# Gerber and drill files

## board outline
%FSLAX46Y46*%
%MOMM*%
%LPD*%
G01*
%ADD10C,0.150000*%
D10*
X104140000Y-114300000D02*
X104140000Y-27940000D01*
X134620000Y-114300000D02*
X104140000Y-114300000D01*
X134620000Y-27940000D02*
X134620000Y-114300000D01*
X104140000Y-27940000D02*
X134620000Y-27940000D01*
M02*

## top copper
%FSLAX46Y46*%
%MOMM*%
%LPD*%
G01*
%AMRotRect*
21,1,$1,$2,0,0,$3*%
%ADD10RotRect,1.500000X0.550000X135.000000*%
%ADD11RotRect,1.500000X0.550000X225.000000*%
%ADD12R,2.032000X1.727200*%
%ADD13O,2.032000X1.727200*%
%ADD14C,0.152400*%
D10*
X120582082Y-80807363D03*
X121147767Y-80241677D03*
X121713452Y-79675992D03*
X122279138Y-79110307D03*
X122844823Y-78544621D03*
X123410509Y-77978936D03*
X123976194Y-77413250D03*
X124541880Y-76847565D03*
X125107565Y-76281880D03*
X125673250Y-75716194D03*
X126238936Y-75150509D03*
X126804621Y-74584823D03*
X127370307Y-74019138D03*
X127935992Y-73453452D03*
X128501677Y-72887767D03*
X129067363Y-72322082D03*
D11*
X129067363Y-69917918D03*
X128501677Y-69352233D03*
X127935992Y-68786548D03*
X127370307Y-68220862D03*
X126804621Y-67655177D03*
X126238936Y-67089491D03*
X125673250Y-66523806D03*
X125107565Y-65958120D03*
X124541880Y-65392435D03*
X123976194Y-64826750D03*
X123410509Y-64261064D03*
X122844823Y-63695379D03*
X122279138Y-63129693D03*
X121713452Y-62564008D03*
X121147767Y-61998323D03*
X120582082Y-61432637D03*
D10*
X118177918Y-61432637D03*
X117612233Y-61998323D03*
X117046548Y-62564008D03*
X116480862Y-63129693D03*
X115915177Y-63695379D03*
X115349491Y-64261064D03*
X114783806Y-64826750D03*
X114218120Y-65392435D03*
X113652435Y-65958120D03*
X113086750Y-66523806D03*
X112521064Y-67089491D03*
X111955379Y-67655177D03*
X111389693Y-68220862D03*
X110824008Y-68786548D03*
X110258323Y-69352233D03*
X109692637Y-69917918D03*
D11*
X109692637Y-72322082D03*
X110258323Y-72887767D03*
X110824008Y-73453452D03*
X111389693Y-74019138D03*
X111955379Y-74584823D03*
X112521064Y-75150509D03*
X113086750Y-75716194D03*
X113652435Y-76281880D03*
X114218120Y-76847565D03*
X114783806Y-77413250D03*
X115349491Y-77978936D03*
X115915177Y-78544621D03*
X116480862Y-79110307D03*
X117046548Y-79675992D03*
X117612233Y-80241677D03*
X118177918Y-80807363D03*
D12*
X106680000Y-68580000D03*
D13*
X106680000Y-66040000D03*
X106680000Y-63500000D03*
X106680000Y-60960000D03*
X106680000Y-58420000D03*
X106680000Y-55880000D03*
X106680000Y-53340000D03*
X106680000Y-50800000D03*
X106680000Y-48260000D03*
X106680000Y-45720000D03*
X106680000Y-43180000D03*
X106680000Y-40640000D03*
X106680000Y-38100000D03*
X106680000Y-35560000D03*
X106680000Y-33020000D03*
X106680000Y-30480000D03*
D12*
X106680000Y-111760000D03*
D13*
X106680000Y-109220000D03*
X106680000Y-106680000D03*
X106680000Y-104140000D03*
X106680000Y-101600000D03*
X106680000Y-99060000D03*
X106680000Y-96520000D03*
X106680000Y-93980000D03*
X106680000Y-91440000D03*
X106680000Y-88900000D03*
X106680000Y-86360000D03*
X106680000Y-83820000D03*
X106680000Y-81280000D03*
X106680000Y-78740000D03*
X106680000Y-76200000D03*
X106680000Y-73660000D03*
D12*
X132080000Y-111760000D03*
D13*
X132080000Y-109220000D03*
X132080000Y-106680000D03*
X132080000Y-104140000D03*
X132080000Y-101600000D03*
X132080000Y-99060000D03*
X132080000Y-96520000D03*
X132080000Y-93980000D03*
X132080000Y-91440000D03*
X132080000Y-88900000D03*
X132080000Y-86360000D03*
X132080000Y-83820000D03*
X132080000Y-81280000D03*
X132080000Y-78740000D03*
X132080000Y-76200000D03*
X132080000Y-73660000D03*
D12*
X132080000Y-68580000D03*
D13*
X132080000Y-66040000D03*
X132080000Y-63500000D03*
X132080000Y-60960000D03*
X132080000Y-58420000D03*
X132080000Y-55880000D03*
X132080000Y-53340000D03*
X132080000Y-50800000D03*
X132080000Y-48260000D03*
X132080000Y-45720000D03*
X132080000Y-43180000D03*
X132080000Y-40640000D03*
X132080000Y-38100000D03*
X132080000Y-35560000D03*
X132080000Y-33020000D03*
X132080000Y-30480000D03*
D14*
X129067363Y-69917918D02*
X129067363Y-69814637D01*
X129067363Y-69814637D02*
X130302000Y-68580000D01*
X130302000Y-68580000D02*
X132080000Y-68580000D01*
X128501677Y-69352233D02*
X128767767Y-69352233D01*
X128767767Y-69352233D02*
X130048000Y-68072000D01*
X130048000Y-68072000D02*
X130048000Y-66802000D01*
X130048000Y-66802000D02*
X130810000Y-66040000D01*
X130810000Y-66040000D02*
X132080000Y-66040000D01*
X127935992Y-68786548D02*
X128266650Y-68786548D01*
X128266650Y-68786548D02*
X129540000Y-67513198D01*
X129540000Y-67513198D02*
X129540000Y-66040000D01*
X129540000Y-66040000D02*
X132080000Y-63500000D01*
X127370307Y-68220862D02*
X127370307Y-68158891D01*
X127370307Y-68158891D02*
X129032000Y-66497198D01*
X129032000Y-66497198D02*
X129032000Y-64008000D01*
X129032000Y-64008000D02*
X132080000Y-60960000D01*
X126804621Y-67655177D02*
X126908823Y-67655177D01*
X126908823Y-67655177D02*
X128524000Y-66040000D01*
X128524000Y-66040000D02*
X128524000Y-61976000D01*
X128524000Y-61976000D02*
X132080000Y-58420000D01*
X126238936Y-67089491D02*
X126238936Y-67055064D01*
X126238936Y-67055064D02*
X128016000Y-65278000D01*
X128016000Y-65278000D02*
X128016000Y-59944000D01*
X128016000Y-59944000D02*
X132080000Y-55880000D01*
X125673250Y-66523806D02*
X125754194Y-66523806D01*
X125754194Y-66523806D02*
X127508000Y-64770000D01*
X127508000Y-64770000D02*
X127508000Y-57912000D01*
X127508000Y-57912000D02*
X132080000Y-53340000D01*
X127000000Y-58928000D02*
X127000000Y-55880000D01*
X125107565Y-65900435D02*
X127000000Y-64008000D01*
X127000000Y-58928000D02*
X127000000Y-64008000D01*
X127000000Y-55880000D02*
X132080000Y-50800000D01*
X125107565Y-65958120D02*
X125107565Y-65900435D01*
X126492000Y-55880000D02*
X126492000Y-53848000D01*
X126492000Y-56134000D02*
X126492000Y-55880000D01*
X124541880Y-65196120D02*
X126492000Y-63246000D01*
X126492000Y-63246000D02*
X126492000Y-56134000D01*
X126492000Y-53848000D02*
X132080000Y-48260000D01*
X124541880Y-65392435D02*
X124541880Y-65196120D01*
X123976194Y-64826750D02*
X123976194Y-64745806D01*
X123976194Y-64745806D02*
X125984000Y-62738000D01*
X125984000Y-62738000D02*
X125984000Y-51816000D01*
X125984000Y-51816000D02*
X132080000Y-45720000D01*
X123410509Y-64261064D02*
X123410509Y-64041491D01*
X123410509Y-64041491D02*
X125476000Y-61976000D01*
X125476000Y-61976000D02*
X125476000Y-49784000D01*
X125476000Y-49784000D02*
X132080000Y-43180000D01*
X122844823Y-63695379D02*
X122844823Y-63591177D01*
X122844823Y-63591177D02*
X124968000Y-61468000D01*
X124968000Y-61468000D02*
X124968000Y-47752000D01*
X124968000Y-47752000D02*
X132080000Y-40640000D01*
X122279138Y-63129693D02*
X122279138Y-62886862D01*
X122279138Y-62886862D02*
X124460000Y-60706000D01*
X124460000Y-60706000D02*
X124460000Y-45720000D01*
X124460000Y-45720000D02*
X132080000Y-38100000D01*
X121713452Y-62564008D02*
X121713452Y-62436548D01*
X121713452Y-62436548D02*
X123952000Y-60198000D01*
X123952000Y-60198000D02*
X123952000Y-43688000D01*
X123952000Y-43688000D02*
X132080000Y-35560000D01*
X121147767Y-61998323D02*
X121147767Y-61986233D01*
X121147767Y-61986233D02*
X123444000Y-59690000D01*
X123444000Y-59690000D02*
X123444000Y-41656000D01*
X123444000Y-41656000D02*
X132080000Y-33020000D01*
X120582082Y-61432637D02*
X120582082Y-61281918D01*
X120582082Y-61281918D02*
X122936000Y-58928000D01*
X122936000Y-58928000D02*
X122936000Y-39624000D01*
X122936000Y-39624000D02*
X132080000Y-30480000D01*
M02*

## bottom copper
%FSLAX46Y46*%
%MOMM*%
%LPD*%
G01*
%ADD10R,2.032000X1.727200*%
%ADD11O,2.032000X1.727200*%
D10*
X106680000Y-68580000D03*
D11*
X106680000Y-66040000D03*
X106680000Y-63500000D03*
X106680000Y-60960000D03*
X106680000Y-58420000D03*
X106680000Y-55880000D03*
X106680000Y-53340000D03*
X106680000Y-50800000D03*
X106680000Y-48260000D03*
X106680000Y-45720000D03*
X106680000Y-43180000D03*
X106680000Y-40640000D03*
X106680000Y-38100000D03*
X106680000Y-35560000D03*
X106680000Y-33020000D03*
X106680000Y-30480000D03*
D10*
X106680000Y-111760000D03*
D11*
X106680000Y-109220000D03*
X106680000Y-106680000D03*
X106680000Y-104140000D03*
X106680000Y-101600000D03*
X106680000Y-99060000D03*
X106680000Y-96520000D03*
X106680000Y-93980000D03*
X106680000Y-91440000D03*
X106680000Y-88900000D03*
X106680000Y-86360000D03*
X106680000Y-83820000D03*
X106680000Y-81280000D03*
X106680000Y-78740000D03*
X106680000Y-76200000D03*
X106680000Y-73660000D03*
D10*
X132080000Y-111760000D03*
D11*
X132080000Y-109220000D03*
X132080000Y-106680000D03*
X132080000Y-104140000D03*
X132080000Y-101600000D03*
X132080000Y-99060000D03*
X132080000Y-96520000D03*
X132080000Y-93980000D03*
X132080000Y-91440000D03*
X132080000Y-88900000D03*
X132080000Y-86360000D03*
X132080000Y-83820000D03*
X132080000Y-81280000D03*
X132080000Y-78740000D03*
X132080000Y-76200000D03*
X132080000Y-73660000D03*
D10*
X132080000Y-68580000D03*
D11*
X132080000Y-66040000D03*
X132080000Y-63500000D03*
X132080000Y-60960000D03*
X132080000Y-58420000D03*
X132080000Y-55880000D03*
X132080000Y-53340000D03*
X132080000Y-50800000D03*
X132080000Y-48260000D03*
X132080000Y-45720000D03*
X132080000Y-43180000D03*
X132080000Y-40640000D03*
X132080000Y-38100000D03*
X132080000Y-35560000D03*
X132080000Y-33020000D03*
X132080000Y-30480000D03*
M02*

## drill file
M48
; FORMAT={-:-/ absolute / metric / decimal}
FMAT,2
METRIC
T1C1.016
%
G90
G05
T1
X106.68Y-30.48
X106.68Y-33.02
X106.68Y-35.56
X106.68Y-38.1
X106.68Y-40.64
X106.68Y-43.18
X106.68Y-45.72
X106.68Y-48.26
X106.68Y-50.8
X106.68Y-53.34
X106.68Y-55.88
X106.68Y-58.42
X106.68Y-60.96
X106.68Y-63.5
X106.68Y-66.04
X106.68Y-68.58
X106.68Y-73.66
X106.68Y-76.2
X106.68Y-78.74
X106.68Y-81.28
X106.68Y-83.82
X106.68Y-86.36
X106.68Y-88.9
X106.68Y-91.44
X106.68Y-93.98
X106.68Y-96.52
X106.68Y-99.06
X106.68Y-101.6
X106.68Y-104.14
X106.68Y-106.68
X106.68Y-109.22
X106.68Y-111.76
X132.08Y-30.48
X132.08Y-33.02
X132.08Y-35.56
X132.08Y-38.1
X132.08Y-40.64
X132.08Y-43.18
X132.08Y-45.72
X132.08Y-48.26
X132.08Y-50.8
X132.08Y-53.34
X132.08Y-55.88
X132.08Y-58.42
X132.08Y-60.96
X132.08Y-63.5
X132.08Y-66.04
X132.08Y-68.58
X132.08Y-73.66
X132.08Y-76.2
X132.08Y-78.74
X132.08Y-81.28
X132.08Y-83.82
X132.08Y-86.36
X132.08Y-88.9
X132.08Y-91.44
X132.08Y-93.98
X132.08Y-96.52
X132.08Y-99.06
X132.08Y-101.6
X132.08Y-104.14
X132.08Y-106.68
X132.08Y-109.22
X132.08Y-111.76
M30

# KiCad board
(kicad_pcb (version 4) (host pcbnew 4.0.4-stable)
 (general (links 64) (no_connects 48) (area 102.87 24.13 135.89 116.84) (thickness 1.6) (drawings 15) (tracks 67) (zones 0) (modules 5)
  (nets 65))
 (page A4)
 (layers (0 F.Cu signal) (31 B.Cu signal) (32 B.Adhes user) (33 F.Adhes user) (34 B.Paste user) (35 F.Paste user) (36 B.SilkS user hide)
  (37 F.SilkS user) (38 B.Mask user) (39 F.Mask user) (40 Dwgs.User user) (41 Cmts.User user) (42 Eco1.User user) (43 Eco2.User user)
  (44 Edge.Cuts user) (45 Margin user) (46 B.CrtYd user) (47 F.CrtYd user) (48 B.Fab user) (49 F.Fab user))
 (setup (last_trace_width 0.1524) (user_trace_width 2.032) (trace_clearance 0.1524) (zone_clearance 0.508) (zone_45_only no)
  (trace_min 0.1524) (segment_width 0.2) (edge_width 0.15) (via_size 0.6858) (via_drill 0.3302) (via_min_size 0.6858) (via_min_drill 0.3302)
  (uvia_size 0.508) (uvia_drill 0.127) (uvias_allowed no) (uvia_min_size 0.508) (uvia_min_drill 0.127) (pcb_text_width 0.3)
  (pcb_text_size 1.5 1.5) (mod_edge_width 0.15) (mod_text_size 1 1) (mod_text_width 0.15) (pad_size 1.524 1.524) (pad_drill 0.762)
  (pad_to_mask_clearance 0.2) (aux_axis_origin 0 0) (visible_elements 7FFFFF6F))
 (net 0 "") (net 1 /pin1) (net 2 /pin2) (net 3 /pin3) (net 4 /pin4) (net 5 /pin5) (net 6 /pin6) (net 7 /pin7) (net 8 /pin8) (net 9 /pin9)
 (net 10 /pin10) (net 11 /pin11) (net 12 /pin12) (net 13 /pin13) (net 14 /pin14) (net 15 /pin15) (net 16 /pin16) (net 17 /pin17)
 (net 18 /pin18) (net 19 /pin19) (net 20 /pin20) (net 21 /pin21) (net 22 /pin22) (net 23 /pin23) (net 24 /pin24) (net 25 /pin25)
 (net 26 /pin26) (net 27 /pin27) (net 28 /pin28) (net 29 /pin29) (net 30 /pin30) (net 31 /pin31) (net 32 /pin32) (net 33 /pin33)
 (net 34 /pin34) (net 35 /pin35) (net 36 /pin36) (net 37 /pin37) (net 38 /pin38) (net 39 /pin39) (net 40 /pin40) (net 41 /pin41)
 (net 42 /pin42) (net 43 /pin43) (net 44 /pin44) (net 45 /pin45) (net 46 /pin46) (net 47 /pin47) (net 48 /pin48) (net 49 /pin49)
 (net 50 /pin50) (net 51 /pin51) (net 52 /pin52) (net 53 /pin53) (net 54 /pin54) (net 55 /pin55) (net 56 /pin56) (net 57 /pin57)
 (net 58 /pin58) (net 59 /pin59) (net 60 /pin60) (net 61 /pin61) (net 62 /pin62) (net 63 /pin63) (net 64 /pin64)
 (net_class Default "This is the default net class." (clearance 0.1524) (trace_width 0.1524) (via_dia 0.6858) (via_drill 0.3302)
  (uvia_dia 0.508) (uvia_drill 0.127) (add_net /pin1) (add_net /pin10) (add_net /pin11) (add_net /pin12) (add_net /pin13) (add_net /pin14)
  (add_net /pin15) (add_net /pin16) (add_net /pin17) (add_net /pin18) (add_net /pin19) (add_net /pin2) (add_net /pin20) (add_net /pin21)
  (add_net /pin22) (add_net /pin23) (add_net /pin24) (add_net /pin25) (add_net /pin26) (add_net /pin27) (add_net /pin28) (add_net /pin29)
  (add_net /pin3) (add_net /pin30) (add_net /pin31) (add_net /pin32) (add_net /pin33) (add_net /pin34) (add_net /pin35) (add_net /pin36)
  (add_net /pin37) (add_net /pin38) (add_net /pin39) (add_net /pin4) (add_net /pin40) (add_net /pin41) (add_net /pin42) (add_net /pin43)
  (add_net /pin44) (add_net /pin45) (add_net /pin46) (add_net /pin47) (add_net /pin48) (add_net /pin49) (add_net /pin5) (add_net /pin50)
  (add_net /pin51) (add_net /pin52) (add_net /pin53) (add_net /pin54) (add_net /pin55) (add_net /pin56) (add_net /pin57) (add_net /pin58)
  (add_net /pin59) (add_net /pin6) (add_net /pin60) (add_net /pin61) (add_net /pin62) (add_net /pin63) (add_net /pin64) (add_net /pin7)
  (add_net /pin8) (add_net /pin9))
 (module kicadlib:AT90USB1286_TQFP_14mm (layer F.Cu) (at 119.38 71.12 135)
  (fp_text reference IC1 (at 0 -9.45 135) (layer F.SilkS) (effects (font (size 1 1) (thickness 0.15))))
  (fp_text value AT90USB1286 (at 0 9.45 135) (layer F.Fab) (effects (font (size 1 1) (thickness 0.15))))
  (pad 1 smd rect (at -7.7 -6 135) (size 1.5 0.55) (layers F.Cu F.Paste F.Mask) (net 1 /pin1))
  (pad 2 smd rect (at -7.7 -5.2 135) (size 1.5 0.55) (layers F.Cu F.Paste F.Mask) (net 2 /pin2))
  (pad 3 smd rect (at -7.7 -4.4 135) (size 1.5 0.55) (layers F.Cu F.Paste F.Mask) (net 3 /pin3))
  (pad 4 smd rect (at -7.7 -3.6 135) (size 1.5 0.55) (layers F.Cu F.Paste F.Mask) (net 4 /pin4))
  (pad 5 smd rect (at -7.7 -2.8 135) (size 1.5 0.55) (layers F.Cu F.Paste F.Mask) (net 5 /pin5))
  (pad 6 smd rect (at -7.7 -2 135) (size 1.5 0.55) (layers F.Cu F.Paste F.Mask) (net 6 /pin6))
  (pad 7 smd rect (at -7.7 -1.2 135) (size 1.5 0.55) (layers F.Cu F.Paste F.Mask) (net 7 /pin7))
  (pad 8 smd rect (at -7.7 -0.4 135) (size 1.5 0.55) (layers F.Cu F.Paste F.Mask) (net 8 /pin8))
  (pad 9 smd rect (at -7.7 0.4 135) (size 1.5 0.55) (layers F.Cu F.Paste F.Mask) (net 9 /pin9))
  (pad 10 smd rect (at -7.7 1.2 135) (size 1.5 0.55) (layers F.Cu F.Paste F.Mask) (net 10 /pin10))
  (pad 11 smd rect (at -7.7 2 135) (size 1.5 0.55) (layers F.Cu F.Paste F.Mask) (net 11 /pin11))
  (pad 12 smd rect (at -7.7 2.8 135) (size 1.5 0.55) (layers F.Cu F.Paste F.Mask) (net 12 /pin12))
  (pad 13 smd rect (at -7.7 3.6 135) (size 1.5 0.55) (layers F.Cu F.Paste F.Mask) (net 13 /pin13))
  (pad 14 smd rect (at -7.7 4.4 135) (size 1.5 0.55) (layers F.Cu F.Paste F.Mask) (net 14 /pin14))
  (pad 15 smd rect (at -7.7 5.2 135) (size 1.5 0.55) (layers F.Cu F.Paste F.Mask) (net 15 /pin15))
  (pad 16 smd rect (at -7.7 6 135) (size 1.5 0.55) (layers F.Cu F.Paste F.Mask) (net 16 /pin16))
  (pad 17 smd rect (at -6 7.7 225) (size 1.5 0.55) (layers F.Cu F.Paste F.Mask) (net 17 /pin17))
  (pad 18 smd rect (at -5.2 7.7 225) (size 1.5 0.55) (layers F.Cu F.Paste F.Mask) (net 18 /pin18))
  (pad 19 smd rect (at -4.4 7.7 225) (size 1.5 0.55) (layers F.Cu F.Paste F.Mask) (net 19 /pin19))
  (pad 20 smd rect (at -3.6 7.7 225) (size 1.5 0.55) (layers F.Cu F.Paste F.Mask) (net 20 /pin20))
  (pad 21 smd rect (at -2.8 7.7 225) (size 1.5 0.55) (layers F.Cu F.Paste F.Mask) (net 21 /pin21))
  (pad 22 smd rect (at -2 7.7 225) (size 1.5 0.55) (layers F.Cu F.Paste F.Mask) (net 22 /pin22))
  (pad 23 smd rect (at -1.2 7.7 225) (size 1.5 0.55) (layers F.Cu F.Paste F.Mask) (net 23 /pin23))
  (pad 24 smd rect (at -0.4 7.7 225) (size 1.5 0.55) (layers F.Cu F.Paste F.Mask) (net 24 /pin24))
  (pad 25 smd rect (at 0.4 7.7 225) (size 1.5 0.55) (layers F.Cu F.Paste F.Mask) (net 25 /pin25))
  (pad 26 smd rect (at 1.2 7.7 225) (size 1.5 0.55) (layers F.Cu F.Paste F.Mask) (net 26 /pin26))
  (pad 27 smd rect (at 2 7.7 225) (size 1.5 0.55) (layers F.Cu F.Paste F.Mask) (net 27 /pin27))
  (pad 28 smd rect (at 2.8 7.7 225) (size 1.5 0.55) (layers F.Cu F.Paste F.Mask) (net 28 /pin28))
  (pad 29 smd rect (at 3.6 7.7 225) (size 1.5 0.55) (layers F.Cu F.Paste F.Mask) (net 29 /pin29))
  (pad 30 smd rect (at 4.4 7.7 225) (size 1.5 0.55) (layers F.Cu F.Paste F.Mask) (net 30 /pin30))
  (pad 31 smd rect (at 5.2 7.7 225) (size 1.5 0.55) (layers F.Cu F.Paste F.Mask) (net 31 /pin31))
  (pad 32 smd rect (at 6 7.7 225) (size 1.5 0.55) (layers F.Cu F.Paste F.Mask) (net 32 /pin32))
  (pad 33 smd rect (at 7.7 6 135) (size 1.5 0.55) (layers F.Cu F.Paste F.Mask) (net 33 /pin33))
  (pad 34 smd rect (at 7.7 5.2 135) (size 1.5 0.55) (layers F.Cu F.Paste F.Mask) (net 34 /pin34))
  (pad 35 smd rect (at 7.7 4.4 135) (size 1.5 0.55) (layers F.Cu F.Paste F.Mask) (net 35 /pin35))
  (pad 36 smd rect (at 7.7 3.6 135) (size 1.5 0.55) (layers F.Cu F.Paste F.Mask) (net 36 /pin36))
  (pad 37 smd rect (at 7.7 2.8 135) (size 1.5 0.55) (layers F.Cu F.Paste F.Mask) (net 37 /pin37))
  (pad 38 smd rect (at 7.7 2 135) (size 1.5 0.55) (layers F.Cu F.Paste F.Mask) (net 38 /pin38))
  (pad 39 smd rect (at 7.7 1.2 135) (size 1.5 0.55) (layers F.Cu F.Paste F.Mask) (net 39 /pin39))
  (pad 40 smd rect (at 7.7 0.4 135) (size 1.5 0.55) (layers F.Cu F.Paste F.Mask) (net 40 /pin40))
  (pad 41 smd rect (at 7.7 -0.4 135) (size 1.5 0.55) (layers F.Cu F.Paste F.Mask) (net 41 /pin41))
  (pad 42 smd rect (at 7.7 -1.2 135) (size 1.5 0.55) (layers F.Cu F.Paste F.Mask) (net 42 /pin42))
  (pad 43 smd rect (at 7.7 -2 135) (size 1.5 0.55) (layers F.Cu F.Paste F.Mask) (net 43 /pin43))
  (pad 44 smd rect (at 7.7 -2.8 135) (size 1.5 0.55) (layers F.Cu F.Paste F.Mask) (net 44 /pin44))
  (pad 45 smd rect (at 7.7 -3.6 135) (size 1.5 0.55) (layers F.Cu F.Paste F.Mask) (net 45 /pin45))
  (pad 46 smd rect (at 7.7 -4.4 135) (size 1.5 0.55) (layers F.Cu F.Paste F.Mask) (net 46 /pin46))
  (pad 47 smd rect (at 7.7 -5.2 135) (size 1.5 0.55) (layers F.Cu F.Paste F.Mask) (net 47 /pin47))
  (pad 48 smd rect (at 7.7 -6 135) (size 1.5 0.55) (layers F.Cu F.Paste F.Mask) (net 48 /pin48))
  (pad 49 smd rect (at 6 -7.7 225) (size 1.5 0.55) (layers F.Cu F.Paste F.Mask) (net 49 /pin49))
  (pad 50 smd rect (at 5.2 -7.7 225) (size 1.5 0.55) (layers F.Cu F.Paste F.Mask) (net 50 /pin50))
  (pad 51 smd rect (at 4.4 -7.7 225) (size 1.5 0.55) (layers F.Cu F.Paste F.Mask) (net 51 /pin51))
  (pad 52 smd rect (at 3.6 -7.7 225) (size 1.5 0.55) (layers F.Cu F.Paste F.Mask) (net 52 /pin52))
  (pad 53 smd rect (at 2.8 -7.7 225) (size 1.5 0.55) (layers F.Cu F.Paste F.Mask) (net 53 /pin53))
  (pad 54 smd rect (at 2 -7.7 225) (size 1.5 0.55) (layers F.Cu F.Paste F.Mask) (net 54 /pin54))
  (pad 55 smd rect (at 1.2 -7.7 225) (size 1.5 0.55) (layers F.Cu F.Paste F.Mask) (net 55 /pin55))
  (pad 56 smd rect (at 0.4 -7.7 225) (size 1.5 0.55) (layers F.Cu F.Paste F.Mask) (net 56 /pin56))
  (pad 57 smd rect (at -0.4 -7.7 225) (size 1.5 0.55) (layers F.Cu F.Paste F.Mask) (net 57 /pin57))
  (pad 58 smd rect (at -1.2 -7.7 225) (size 1.5 0.55) (layers F.Cu F.Paste F.Mask) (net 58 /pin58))
  (pad 59 smd rect (at -2 -7.7 225) (size 1.5 0.55) (layers F.Cu F.Paste F.Mask) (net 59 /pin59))
  (pad 60 smd rect (at -2.8 -7.7 225) (size 1.5 0.55) (layers F.Cu F.Paste F.Mask) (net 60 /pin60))
  (pad 61 smd rect (at -3.6 -7.7 225) (size 1.5 0.55) (layers F.Cu F.Paste F.Mask) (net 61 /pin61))
  (pad 62 smd rect (at -4.4 -7.7 225) (size 1.5 0.55) (layers F.Cu F.Paste F.Mask) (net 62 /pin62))
  (pad 63 smd rect (at -5.2 -7.7 225) (size 1.5 0.55) (layers F.Cu F.Paste F.Mask) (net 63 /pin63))
  (pad 64 smd rect (at -6 -7.7 225) (size 1.5 0.55) (layers F.Cu F.Paste F.Mask) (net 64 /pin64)))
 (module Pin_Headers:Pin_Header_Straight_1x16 (layer F.Cu) (at 106.68 68.58 180)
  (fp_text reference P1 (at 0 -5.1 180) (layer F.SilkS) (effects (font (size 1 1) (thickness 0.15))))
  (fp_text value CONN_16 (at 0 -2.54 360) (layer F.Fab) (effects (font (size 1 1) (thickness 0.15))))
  (pad 1 thru_hole rect (at 0 0 180) (size 2.032 1.7272) (drill 1.016) (layers *.Cu *.Mask) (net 48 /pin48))
  (pad 2 thru_hole oval (at 0 2.54 180) (size 2.032 1.7272) (drill 1.016) (layers *.Cu *.Mask) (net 47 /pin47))
  (pad 3 thru_hole oval (at 0 5.08 180) (size 2.032 1.7272) (drill 1.016) (layers *.Cu *.Mask) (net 46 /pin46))
  (pad 4 thru_hole oval (at 0 7.62 180) (size 2.032 1.7272) (drill 1.016) (layers *.Cu *.Mask) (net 45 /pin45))
  (pad 5 thru_hole oval (at 0 10.16 180) (size 2.032 1.7272) (drill 1.016) (layers *.Cu *.Mask) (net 44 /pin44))
  (pad 6 thru_hole oval (at 0 12.7 180) (size 2.032 1.7272) (drill 1.016) (layers *.Cu *.Mask) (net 43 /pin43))
  (pad 7 thru_hole oval (at 0 15.24 180) (size 2.032 1.7272) (drill 1.016) (layers *.Cu *.Mask) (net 42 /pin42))
  (pad 8 thru_hole oval (at 0 17.78 180) (size 2.032 1.7272) (drill 1.016) (layers *.Cu *.Mask) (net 41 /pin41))
  (pad 9 thru_hole oval (at 0 20.32 180) (size 2.032 1.7272) (drill 1.016) (layers *.Cu *.Mask) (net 40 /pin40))
  (pad 10 thru_hole oval (at 0 22.86 180) (size 2.032 1.7272) (drill 1.016) (layers *.Cu *.Mask) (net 39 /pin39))
  (pad 11 thru_hole oval (at 0 25.4 180) (size 2.032 1.7272) (drill 1.016) (layers *.Cu *.Mask) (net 38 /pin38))
  (pad 12 thru_hole oval (at 0 27.94 180) (size 2.032 1.7272) (drill 1.016) (layers *.Cu *.Mask) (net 37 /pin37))
  (pad 13 thru_hole oval (at 0 30.48 180) (size 2.032 1.7272) (drill 1.016) (layers *.Cu *.Mask) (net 36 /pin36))
  (pad 14 thru_hole oval (at 0 33.02 180) (size 2.032 1.7272) (drill 1.016) (layers *.Cu *.Mask) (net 35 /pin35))
  (pad 15 thru_hole oval (at 0 35.56 180) (size 2.032 1.7272) (drill 1.016) (layers *.Cu *.Mask) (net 34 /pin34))
  (pad 16 thru_hole oval (at 0 38.1 180) (size 2.032 1.7272) (drill 1.016) (layers *.Cu *.Mask) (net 33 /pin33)))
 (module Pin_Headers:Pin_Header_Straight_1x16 (layer F.Cu) (at 106.68 111.76 180)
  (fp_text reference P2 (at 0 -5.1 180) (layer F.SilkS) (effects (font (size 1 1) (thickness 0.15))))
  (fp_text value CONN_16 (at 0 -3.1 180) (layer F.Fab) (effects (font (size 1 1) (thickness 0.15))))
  (pad 1 thru_hole rect (at 0 0 180) (size 2.032 1.7272) (drill 1.016) (layers *.Cu *.Mask) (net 64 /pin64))
  (pad 2 thru_hole oval (at 0 2.54 180) (size 2.032 1.7272) (drill 1.016) (layers *.Cu *.Mask) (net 63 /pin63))
  (pad 3 thru_hole oval (at 0 5.08 180) (size 2.032 1.7272) (drill 1.016) (layers *.Cu *.Mask) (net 62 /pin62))
  (pad 4 thru_hole oval (at 0 7.62 180) (size 2.032 1.7272) (drill 1.016) (layers *.Cu *.Mask) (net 61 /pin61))
  (pad 5 thru_hole oval (at 0 10.16 180) (size 2.032 1.7272) (drill 1.016) (layers *.Cu *.Mask) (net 60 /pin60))
  (pad 6 thru_hole oval (at 0 12.7 180) (size 2.032 1.7272) (drill 1.016) (layers *.Cu *.Mask) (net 59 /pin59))
  (pad 7 thru_hole oval (at 0 15.24 180) (size 2.032 1.7272) (drill 1.016) (layers *.Cu *.Mask) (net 58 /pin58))
  (pad 8 thru_hole oval (at 0 17.78 180) (size 2.032 1.7272) (drill 1.016) (layers *.Cu *.Mask) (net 57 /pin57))
  (pad 9 thru_hole oval (at 0 20.32 180) (size 2.032 1.7272) (drill 1.016) (layers *.Cu *.Mask) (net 56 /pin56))
  (pad 10 thru_hole oval (at 0 22.86 180) (size 2.032 1.7272) (drill 1.016) (layers *.Cu *.Mask) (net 55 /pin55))
  (pad 11 thru_hole oval (at 0 25.4 180) (size 2.032 1.7272) (drill 1.016) (layers *.Cu *.Mask) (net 54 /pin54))
  (pad 12 thru_hole oval (at 0 27.94 180) (size 2.032 1.7272) (drill 1.016) (layers *.Cu *.Mask) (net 53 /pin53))
  (pad 13 thru_hole oval (at 0 30.48 180) (size 2.032 1.7272) (drill 1.016) (layers *.Cu *.Mask) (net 52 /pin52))
  (pad 14 thru_hole oval (at 0 33.02 180) (size 2.032 1.7272) (drill 1.016) (layers *.Cu *.Mask) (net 51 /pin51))
  (pad 15 thru_hole oval (at 0 35.56 180) (size 2.032 1.7272) (drill 1.016) (layers *.Cu *.Mask) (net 50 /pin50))
  (pad 16 thru_hole oval (at 0 38.1 180) (size 2.032 1.7272) (drill 1.016) (layers *.Cu *.Mask) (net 49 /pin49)))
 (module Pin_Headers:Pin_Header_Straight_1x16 (layer F.Cu) (at 132.08 111.76 180)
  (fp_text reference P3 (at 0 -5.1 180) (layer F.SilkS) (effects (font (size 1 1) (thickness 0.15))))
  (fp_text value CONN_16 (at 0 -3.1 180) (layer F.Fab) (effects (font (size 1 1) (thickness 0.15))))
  (pad 1 thru_hole rect (at 0 0 180) (size 2.032 1.7272) (drill 1.016) (layers *.Cu *.Mask) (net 1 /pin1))
  (pad 2 thru_hole oval (at 0 2.54 180) (size 2.032 1.7272) (drill 1.016) (layers *.Cu *.Mask) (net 2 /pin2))
  (pad 3 thru_hole oval (at 0 5.08 180) (size 2.032 1.7272) (drill 1.016) (layers *.Cu *.Mask) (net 3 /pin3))
  (pad 4 thru_hole oval (at 0 7.62 180) (size 2.032 1.7272) (drill 1.016) (layers *.Cu *.Mask) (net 4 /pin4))
  (pad 5 thru_hole oval (at 0 10.16 180) (size 2.032 1.7272) (drill 1.016) (layers *.Cu *.Mask) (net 5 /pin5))
  (pad 6 thru_hole oval (at 0 12.7 180) (size 2.032 1.7272) (drill 1.016) (layers *.Cu *.Mask) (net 6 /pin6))
  (pad 7 thru_hole oval (at 0 15.24 180) (size 2.032 1.7272) (drill 1.016) (layers *.Cu *.Mask) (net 7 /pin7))
  (pad 8 thru_hole oval (at 0 17.78 180) (size 2.032 1.7272) (drill 1.016) (layers *.Cu *.Mask) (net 8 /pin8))
  (pad 9 thru_hole oval (at 0 20.32 180) (size 2.032 1.7272) (drill 1.016) (layers *.Cu *.Mask) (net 9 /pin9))
  (pad 10 thru_hole oval (at 0 22.86 180) (size 2.032 1.7272) (drill 1.016) (layers *.Cu *.Mask) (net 10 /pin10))
  (pad 11 thru_hole oval (at 0 25.4 180) (size 2.032 1.7272) (drill 1.016) (layers *.Cu *.Mask) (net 11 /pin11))
  (pad 12 thru_hole oval (at 0 27.94 180) (size 2.032 1.7272) (drill 1.016) (layers *.Cu *.Mask) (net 12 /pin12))
  (pad 13 thru_hole oval (at 0 30.48 180) (size 2.032 1.7272) (drill 1.016) (layers *.Cu *.Mask) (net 13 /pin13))
  (pad 14 thru_hole oval (at 0 33.02 180) (size 2.032 1.7272) (drill 1.016) (layers *.Cu *.Mask) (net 14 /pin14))
  (pad 15 thru_hole oval (at 0 35.56 180) (size 2.032 1.7272) (drill 1.016) (layers *.Cu *.Mask) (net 15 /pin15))
  (pad 16 thru_hole oval (at 0 38.1 180) (size 2.032 1.7272) (drill 1.016) (layers *.Cu *.Mask) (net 16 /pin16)))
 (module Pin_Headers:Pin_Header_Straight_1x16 (layer F.Cu) (at 132.08 68.58 180)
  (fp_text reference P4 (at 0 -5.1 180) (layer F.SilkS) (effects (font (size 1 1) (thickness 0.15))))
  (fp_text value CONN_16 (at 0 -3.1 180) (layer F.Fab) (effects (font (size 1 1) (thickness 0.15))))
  (pad 1 thru_hole rect (at 0 0 180) (size 2.032 1.7272) (drill 1.016) (layers *.Cu *.Mask) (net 17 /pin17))
  (pad 2 thru_hole oval (at 0 2.54 180) (size 2.032 1.7272) (drill 1.016) (layers *.Cu *.Mask) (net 18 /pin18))
  (pad 3 thru_hole oval (at 0 5.08 180) (size 2.032 1.7272) (drill 1.016) (layers *.Cu *.Mask) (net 19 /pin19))
  (pad 4 thru_hole oval (at 0 7.62 180) (size 2.032 1.7272) (drill 1.016) (layers *.Cu *.Mask) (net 20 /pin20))
  (pad 5 thru_hole oval (at 0 10.16 180) (size 2.032 1.7272) (drill 1.016) (layers *.Cu *.Mask) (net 21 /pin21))
  (pad 6 thru_hole oval (at 0 12.7 180) (size 2.032 1.7272) (drill 1.016) (layers *.Cu *.Mask) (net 22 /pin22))
  (pad 7 thru_hole oval (at 0 15.24 180) (size 2.032 1.7272) (drill 1.016) (layers *.Cu *.Mask) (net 23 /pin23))
  (pad 8 thru_hole oval (at 0 17.78 180) (size 2.032 1.7272) (drill 1.016) (layers *.Cu *.Mask) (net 24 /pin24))
  (pad 9 thru_hole oval (at 0 20.32 180) (size 2.032 1.7272) (drill 1.016) (layers *.Cu *.Mask) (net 25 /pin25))
  (pad 10 thru_hole oval (at 0 22.86 180) (size 2.032 1.7272) (drill 1.016) (layers *.Cu *.Mask) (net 26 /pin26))
  (pad 11 thru_hole oval (at 0 25.4 180) (size 2.032 1.7272) (drill 1.016) (layers *.Cu *.Mask) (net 27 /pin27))
  (pad 12 thru_hole oval (at 0 27.94 180) (size 2.032 1.7272) (drill 1.016) (layers *.Cu *.Mask) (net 28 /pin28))
  (pad 13 thru_hole oval (at 0 30.48 180) (size 2.032 1.7272) (drill 1.016) (layers *.Cu *.Mask) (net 29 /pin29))
  (pad 14 thru_hole oval (at 0 33.02 180) (size 2.032 1.7272) (drill 1.016) (layers *.Cu *.Mask) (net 30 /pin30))
  (pad 15 thru_hole oval (at 0 35.56 180) (size 2.032 1.7272) (drill 1.016) (layers *.Cu *.Mask) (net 31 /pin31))
  (pad 16 thru_hole oval (at 0 38.1 180) (size 2.032 1.7272) (drill 1.016) (layers *.Cu *.Mask) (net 32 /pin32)))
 (gr_line (start 104.14 114.3) (end 104.14 27.94) (angle 90) (layer Edge.Cuts) (width 0.15))
 (gr_line (start 134.62 114.3) (end 104.14 114.3) (angle 90) (layer Edge.Cuts) (width 0.15))
 (gr_line (start 134.62 27.94) (end 134.62 114.3) (angle 90) (layer Edge.Cuts) (width 0.15))
 (gr_line (start 104.14 27.94) (end 134.62 27.94) (angle 90) (layer Edge.Cuts) (width 0.15))
 (segment (start 129.067363 69.917918) (end 129.067363 69.814637) (width 0.1524) (layer F.Cu) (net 17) (status C00000))
 (segment (start 129.067363 69.814637) (end 130.302 68.58) (width 0.1524) (layer F.Cu) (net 17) (status 400000))
 (segment (start 130.302 68.58) (end 132.08 68.58) (width 0.1524) (layer F.Cu) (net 17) (status 800000))
 (segment (start 128.501677 69.352233) (end 128.767767 69.352233) (width 0.1524) (layer F.Cu) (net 18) (status C00000))
 (segment (start 128.767767 69.352233) (end 130.048 68.072) (width 0.1524) (layer F.Cu) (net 18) (status 400000))
 (segment (start 130.048 68.072) (end 130.048 66.802) (width 0.1524) (layer F.Cu) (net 18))
 (segment (start 130.048 66.802) (end 130.81 66.04) (width 0.1524) (layer F.Cu) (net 18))
 (segment (start 130.81 66.04) (end 132.08 66.04) (width 0.1524) (layer F.Cu) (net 18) (status 800000))
 (segment (start 127.935992 68.786548) (end 128.26665 68.786548) (width 0.1524) (layer F.Cu) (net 19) (status C00000))
 (segment (start 128.26665 68.786548) (end 129.54 67.513198) (width 0.1524) (layer F.Cu) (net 19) (status 400000))
 (segment (start 129.54 67.513198) (end 129.54 66.04) (width 0.1524) (layer F.Cu) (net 19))
 (segment (start 129.54 66.04) (end 132.08 63.5) (width 0.1524) (layer F.Cu) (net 19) (status 800000))
 (segment (start 127.370307 68.220862) (end 127.370307 68.158891) (width 0.1524) (layer F.Cu) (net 20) (status C00000))
 (segment (start 127.370307 68.158891) (end 129.032 66.497198) (width 0.1524) (layer F.Cu) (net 20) (status 400000))
 (segment (start 129.032 66.497198) (end 129.032 64.008) (width 0.1524) (layer F.Cu) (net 20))
 (segment (start 129.032 64.008) (end 132.08 60.96) (width 0.1524) (layer F.Cu) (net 20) (status 800000))
 (segment (start 126.804621 67.655177) (end 126.908823 67.655177) (width 0.1524) (layer F.Cu) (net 21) (status C00000))
 (segment (start 126.908823 67.655177) (end 128.524 66.04) (width 0.1524) (layer F.Cu) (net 21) (status 400000))
 (segment (start 128.524 66.04) (end 128.524 61.976) (width 0.1524) (layer F.Cu) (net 21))
 (segment (start 128.524 61.976) (end 132.08 58.42) (width 0.1524) (layer F.Cu) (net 21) (status 800000))
 (segment (start 126.238936 67.089491) (end 126.238936 67.055064) (width 0.1524) (layer F.Cu) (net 22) (status C00000))
 (segment (start 126.238936 67.055064) (end 128.016 65.278) (width 0.1524) (layer F.Cu) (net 22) (status 400000))
 (segment (start 128.016 65.278) (end 128.016 59.944) (width 0.1524) (layer F.Cu) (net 22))
 (segment (start 128.016 59.944) (end 132.08 55.88) (width 0.1524) (layer F.Cu) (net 22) (status 800000))
 (segment (start 125.67325 66.523806) (end 125.754194 66.523806) (width 0.1524) (layer F.Cu) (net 23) (status C00000))
 (segment (start 125.754194 66.523806) (end 127.508 64.77) (width 0.1524) (layer F.Cu) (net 23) (status 400000))
 (segment (start 127.508 64.77) (end 127.508 57.912) (width 0.1524) (layer F.Cu) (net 23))
 (segment (start 127.508 57.912) (end 132.08 53.34) (width 0.1524) (layer F.Cu) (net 23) (status 800000))
 (segment (start 127 58.928) (end 127 55.88) (width 0.1524) (layer F.Cu) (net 24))
 (segment (start 125.107565 65.900435) (end 127 64.008) (width 0.1524) (layer F.Cu) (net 24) (status 400000))
 (segment (start 127 58.928) (end 127 64.008) (width 0.1524) (layer F.Cu) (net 24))
 (segment (start 127 55.88) (end 132.08 50.8) (width 0.1524) (layer F.Cu) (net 24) (status 800000))
 (segment (start 125.107565 65.95812) (end 125.107565 65.900435) (width 0.1524) (layer F.Cu) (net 24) (status C00000))
 (segment (start 126.492 55.88) (end 126.492 53.848) (width 0.1524) (layer F.Cu) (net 25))
 (segment (start 126.492 56.134) (end 126.492 55.88) (width 0.1524) (layer F.Cu) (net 25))
 (segment (start 124.54188 65.19612) (end 126.492 63.246) (width 0.1524) (layer F.Cu) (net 25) (status 400000))
 (segment (start 126.492 63.246) (end 126.492 56.134) (width 0.1524) (layer F.Cu) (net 25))
 (segment (start 126.492 53.848) (end 132.08 48.26) (width 0.1524) (layer F.Cu) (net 25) (status 800000))
 (segment (start 124.54188 65.392435) (end 124.54188 65.19612) (width 0.1524) (layer F.Cu) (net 25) (status C00000))
 (segment (start 123.976194 64.82675) (end 123.976194 64.745806) (width 0.1524) (layer F.Cu) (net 26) (status C00000))
 (segment (start 123.976194 64.745806) (end 125.984 62.738) (width 0.1524) (layer F.Cu) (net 26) (status 400000))
 (segment (start 125.984 62.738) (end 125.984 51.816) (width 0.1524) (layer F.Cu) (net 26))
 (segment (start 125.984 51.816) (end 132.08 45.72) (width 0.1524) (layer F.Cu) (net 26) (status 800000))
 (segment (start 123.410509 64.261064) (end 123.410509 64.041491) (width 0.1524) (layer F.Cu) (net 27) (status C00000))
 (segment (start 123.410509 64.041491) (end 125.476 61.976) (width 0.1524) (layer F.Cu) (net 27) (status 400000))
 (segment (start 125.476 61.976) (end 125.476 49.784) (width 0.1524) (layer F.Cu) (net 27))
 (segment (start 125.476 49.784) (end 132.08 43.18) (width 0.1524) (layer F.Cu) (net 27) (status 800000))
 (segment (start 122.844823 63.695379) (end 122.844823 63.591177) (width 0.1524) (layer F.Cu) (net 28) (status C00000))
 (segment (start 122.844823 63.591177) (end 124.968 61.468) (width 0.1524) (layer F.Cu) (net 28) (status 400000))
 (segment (start 124.968 61.468) (end 124.968 47.752) (width 0.1524) (layer F.Cu) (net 28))
 (segment (start 124.968 47.752) (end 132.08 40.64) (width 0.1524) (layer F.Cu) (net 28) (status 800000))
 (segment (start 122.279138 63.129693) (end 122.279138 62.886862) (width 0.1524) (layer F.Cu) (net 29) (status C00000))
 (segment (start 122.279138 62.886862) (end 124.46 60.706) (width 0.1524) (layer F.Cu) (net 29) (status 400000))
 (segment (start 124.46 60.706) (end 124.46 45.72) (width 0.1524) (layer F.Cu) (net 29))
 (segment (start 124.46 45.72) (end 132.08 38.1) (width 0.1524) (layer F.Cu) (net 29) (status 800000))
 (segment (start 121.713452 62.564008) (end 121.713452 62.436548) (width 0.1524) (layer F.Cu) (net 30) (status C00000))
 (segment (start 121.713452 62.436548) (end 123.952 60.198) (width 0.1524) (layer F.Cu) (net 30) (status 400000))
 (segment (start 123.952 60.198) (end 123.952 43.688) (width 0.1524) (layer F.Cu) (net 30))
 (segment (start 123.952 43.688) (end 132.08 35.56) (width 0.1524) (layer F.Cu) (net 30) (status 800000))
 (segment (start 121.147767 61.998323) (end 121.147767 61.986233) (width 0.1524) (layer F.Cu) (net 31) (status C00000))
 (segment (start 121.147767 61.986233) (end 123.444 59.69) (width 0.1524) (layer F.Cu) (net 31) (status 400000))
 (segment (start 123.444 59.69) (end 123.444 41.656) (width 0.1524) (layer F.Cu) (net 31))
 (segment (start 123.444 41.656) (end 132.08 33.02) (width 0.1524) (layer F.Cu) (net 31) (status 800000))
 (segment (start 120.582082 61.432637) (end 120.582082 61.281918) (width 0.1524) (layer F.Cu) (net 32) (status C00000))
 (segment (start 120.582082 61.281918) (end 122.936 58.928) (width 0.1524) (layer F.Cu) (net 32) (status 400000))
 (segment (start 122.936 58.928) (end 122.936 39.624) (width 0.1524) (layer F.Cu) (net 32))
 (segment (start 122.936 39.624) (end 132.08 30.48) (width 0.1524) (layer F.Cu) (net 32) (status 800000)))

